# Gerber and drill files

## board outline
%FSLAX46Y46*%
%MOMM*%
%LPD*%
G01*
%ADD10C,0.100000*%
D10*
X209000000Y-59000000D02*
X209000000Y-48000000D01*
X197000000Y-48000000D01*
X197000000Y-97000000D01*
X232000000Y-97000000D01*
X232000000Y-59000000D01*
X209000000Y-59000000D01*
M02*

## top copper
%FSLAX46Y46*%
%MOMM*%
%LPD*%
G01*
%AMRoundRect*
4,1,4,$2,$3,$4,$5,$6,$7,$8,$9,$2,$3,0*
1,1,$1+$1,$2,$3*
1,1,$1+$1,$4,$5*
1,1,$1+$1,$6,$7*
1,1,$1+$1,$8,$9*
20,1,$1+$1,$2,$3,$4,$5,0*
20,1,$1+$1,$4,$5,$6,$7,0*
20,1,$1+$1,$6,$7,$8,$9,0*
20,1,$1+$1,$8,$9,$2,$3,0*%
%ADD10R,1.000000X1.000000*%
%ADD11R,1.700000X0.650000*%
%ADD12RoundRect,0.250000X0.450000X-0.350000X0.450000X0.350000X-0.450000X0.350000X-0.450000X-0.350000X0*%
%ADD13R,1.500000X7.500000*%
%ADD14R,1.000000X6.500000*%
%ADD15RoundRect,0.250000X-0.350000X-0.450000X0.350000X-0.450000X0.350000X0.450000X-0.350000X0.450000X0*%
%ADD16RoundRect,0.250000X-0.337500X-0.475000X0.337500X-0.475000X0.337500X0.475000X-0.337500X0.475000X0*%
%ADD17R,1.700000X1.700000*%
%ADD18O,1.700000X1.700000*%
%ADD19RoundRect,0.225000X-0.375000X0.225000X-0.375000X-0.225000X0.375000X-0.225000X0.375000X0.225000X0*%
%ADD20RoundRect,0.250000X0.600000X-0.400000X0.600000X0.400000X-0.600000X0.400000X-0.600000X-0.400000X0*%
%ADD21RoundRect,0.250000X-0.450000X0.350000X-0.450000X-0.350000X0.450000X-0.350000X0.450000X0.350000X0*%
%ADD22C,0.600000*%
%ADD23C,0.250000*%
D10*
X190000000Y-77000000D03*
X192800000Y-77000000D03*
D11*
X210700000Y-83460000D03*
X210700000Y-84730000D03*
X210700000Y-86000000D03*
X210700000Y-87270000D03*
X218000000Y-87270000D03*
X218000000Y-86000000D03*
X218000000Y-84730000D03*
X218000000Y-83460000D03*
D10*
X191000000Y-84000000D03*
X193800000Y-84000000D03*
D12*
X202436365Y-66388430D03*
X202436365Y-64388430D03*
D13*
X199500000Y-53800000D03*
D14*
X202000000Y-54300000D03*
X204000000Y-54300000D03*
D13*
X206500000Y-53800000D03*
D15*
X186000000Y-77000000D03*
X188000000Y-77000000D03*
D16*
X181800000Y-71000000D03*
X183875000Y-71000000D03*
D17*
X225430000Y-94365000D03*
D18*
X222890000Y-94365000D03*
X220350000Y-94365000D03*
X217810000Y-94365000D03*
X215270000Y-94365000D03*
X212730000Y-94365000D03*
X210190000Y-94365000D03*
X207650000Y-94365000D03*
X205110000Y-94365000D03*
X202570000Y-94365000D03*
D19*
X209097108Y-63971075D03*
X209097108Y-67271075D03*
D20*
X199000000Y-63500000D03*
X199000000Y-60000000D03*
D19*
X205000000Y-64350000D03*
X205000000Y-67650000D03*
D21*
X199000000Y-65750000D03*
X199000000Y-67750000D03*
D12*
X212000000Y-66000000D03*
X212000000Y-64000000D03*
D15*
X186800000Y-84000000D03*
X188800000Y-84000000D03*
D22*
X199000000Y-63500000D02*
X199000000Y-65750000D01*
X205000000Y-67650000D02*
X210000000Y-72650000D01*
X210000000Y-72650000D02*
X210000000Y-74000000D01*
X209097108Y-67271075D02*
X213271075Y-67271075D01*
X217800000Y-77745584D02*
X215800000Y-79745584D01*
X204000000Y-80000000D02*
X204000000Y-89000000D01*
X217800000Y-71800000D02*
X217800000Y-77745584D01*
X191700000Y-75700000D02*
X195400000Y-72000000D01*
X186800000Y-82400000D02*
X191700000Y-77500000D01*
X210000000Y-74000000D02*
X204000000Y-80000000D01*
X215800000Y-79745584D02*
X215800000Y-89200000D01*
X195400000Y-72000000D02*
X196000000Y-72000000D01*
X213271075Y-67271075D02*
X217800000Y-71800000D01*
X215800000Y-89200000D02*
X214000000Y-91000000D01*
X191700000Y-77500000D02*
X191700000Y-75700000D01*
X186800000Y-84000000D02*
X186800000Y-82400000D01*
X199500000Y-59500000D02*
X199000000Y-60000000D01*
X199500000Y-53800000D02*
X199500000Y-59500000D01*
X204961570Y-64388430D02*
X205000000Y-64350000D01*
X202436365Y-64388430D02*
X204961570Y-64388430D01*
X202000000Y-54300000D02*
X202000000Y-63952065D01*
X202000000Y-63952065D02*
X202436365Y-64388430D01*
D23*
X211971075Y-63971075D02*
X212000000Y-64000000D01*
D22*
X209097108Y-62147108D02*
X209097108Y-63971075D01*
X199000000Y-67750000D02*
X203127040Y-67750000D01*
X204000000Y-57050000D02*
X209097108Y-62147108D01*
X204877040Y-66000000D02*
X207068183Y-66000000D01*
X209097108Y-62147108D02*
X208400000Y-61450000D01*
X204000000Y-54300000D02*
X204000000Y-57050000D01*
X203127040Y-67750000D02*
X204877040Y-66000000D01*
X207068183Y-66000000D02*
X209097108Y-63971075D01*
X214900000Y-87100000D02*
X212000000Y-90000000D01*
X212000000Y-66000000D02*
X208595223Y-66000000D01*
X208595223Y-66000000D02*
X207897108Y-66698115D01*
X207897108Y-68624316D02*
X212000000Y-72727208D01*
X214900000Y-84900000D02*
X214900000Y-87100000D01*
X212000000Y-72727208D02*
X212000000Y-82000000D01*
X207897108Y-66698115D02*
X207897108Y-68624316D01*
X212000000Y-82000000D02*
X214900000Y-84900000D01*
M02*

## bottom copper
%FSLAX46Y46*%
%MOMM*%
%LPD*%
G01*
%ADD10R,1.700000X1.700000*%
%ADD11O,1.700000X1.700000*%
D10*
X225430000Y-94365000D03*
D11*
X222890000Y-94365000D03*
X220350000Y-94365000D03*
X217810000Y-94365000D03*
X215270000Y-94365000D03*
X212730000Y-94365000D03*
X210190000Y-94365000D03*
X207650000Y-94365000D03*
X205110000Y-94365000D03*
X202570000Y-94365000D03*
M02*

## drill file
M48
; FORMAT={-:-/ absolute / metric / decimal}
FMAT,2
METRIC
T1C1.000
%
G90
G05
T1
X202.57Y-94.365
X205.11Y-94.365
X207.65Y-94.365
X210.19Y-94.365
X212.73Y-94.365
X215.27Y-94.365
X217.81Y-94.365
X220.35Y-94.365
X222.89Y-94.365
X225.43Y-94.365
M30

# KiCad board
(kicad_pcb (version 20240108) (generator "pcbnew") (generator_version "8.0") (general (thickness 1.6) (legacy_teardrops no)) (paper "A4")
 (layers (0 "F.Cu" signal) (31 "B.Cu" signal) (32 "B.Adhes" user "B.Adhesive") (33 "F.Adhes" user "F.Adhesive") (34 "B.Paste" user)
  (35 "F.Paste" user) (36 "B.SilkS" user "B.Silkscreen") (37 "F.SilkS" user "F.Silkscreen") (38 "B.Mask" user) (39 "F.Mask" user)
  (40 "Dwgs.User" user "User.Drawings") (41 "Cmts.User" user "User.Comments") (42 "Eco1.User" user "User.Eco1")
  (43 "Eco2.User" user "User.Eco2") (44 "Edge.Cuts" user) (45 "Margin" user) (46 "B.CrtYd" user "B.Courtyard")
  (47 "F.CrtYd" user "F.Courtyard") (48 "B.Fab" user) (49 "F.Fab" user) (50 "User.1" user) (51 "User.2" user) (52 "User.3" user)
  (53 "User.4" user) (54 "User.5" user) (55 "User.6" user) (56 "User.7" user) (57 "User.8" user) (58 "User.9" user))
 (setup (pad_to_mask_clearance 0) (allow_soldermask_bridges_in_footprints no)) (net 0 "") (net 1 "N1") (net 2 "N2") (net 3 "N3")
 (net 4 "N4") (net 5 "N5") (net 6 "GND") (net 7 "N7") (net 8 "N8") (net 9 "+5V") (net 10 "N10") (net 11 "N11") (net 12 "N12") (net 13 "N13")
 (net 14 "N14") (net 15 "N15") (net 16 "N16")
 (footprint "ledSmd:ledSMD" (layer "F.Cu") (at 191.8 77)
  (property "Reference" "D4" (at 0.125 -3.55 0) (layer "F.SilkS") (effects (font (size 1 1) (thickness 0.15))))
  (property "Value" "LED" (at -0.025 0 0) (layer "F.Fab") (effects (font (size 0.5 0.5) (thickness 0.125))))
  (pad "1" smd rect (at -1.8 0) (size 1 1) (layers "F.Cu" "F.Paste" "F.Mask") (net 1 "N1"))
  (pad "2" smd rect (at 1 0) (size 1 1) (layers "F.Cu" "F.Paste" "F.Mask") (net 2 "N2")))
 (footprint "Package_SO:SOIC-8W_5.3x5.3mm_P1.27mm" (layer "F.Cu") (at 214.35 85.365)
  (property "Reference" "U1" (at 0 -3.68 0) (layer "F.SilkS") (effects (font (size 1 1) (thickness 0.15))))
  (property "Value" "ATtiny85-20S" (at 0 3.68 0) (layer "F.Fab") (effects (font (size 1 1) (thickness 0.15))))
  (pad "1" smd rect (at -3.65 -1.905) (size 1.7 0.65) (layers "F.Cu" "F.Paste" "F.Mask") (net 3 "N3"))
  (pad "2" smd rect (at -3.65 -0.635) (size 1.7 0.65) (layers "F.Cu" "F.Paste" "F.Mask") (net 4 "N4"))
  (pad "3" smd rect (at -3.65 0.635) (size 1.7 0.65) (layers "F.Cu" "F.Paste" "F.Mask") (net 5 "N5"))
  (pad "4" smd rect (at -3.65 1.905) (size 1.7 0.65) (layers "F.Cu" "F.Paste" "F.Mask") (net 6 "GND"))
  (pad "5" smd rect (at 3.65 1.905) (size 1.7 0.65) (layers "F.Cu" "F.Paste" "F.Mask") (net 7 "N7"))
  (pad "6" smd rect (at 3.65 0.635) (size 1.7 0.65) (layers "F.Cu" "F.Paste" "F.Mask") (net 2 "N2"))
  (pad "7" smd rect (at 3.65 -0.635) (size 1.7 0.65) (layers "F.Cu" "F.Paste" "F.Mask") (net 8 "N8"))
  (pad "8" smd rect (at 3.65 -1.905) (size 1.7 0.65) (layers "F.Cu" "F.Paste" "F.Mask") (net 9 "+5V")))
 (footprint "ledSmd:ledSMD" (layer "F.Cu") (at 192.8 84)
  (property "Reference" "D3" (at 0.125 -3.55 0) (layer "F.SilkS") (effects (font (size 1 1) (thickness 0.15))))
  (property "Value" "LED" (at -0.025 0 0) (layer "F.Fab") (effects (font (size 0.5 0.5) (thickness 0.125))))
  (pad "1" smd rect (at -1.8 0) (size 1 1) (layers "F.Cu" "F.Paste" "F.Mask") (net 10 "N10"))
  (pad "2" smd rect (at 1 0) (size 1 1) (layers "F.Cu" "F.Paste" "F.Mask") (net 9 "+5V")))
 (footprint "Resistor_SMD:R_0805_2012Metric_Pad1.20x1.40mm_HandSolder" (layer "F.Cu") (at 202.436365 65.38843 90)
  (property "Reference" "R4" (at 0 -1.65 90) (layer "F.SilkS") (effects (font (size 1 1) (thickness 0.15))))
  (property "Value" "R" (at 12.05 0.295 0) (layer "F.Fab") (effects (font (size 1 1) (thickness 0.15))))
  (pad "1" smd roundrect (at -1 0 90) (size 1.2 1.4) (layers "F.Cu" "F.Paste" "F.Mask") (roundrect_rratio 0.208333) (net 4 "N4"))
  (pad "2" smd roundrect (at 1 0 90) (size 1.2 1.4) (layers "F.Cu" "F.Paste" "F.Mask") (roundrect_rratio 0.208333) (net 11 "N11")))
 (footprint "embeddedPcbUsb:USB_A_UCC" (layer "F.Cu") (at 203 54 -90)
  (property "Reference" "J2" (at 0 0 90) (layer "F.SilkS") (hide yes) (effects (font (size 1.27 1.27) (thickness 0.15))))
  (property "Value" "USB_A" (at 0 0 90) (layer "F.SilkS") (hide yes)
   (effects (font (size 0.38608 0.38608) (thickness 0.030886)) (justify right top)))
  (pad "1" smd rect (at -0.2 3.5 270) (size 7.5 1.5) (layers "F.Cu" "F.Paste" "F.Mask") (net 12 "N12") (solder_mask_margin 0.1016))
  (pad "2" smd rect (at 0.3 1 270) (size 6.5 1) (layers "F.Cu" "F.Paste" "F.Mask") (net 11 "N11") (solder_mask_margin 0.1016))
  (pad "3" smd rect (at 0.3 -1 270) (size 6.5 1) (layers "F.Cu" "F.Paste" "F.Mask") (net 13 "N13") (solder_mask_margin 0.1016))
  (pad "4" smd rect (at -0.2 -3.5 270) (size 7.5 1.5) (layers "F.Cu" "F.Paste" "F.Mask") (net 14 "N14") (solder_mask_margin 0.1016)))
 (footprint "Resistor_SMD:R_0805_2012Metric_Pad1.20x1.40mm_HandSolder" (layer "F.Cu") (at 187 77)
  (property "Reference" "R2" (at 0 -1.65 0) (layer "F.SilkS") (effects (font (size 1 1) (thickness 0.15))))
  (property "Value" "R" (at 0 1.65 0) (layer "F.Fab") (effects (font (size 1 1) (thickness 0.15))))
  (pad "1" smd roundrect (at -1 0) (size 1.2 1.4) (layers "F.Cu" "F.Paste" "F.Mask") (roundrect_rratio 0.208333) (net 6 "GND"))
  (pad "2" smd roundrect (at 1 0) (size 1.2 1.4) (layers "F.Cu" "F.Paste" "F.Mask") (roundrect_rratio 0.208333) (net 1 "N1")))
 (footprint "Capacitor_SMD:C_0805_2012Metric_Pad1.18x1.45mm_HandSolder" (layer "F.Cu") (at 182.8375 71)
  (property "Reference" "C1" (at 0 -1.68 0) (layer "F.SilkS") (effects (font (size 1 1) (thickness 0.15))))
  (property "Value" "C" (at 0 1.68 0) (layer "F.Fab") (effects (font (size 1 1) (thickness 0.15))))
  (pad "1" smd roundrect (at -1.0375 0) (size 1.175 1.45) (layers "F.Cu" "F.Paste" "F.Mask") (roundrect_rratio 0.212766) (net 9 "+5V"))
  (pad "2" smd roundrect (at 1.0375 0) (size 1.175 1.45) (layers "F.Cu" "F.Paste" "F.Mask") (roundrect_rratio 0.212766) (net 6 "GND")))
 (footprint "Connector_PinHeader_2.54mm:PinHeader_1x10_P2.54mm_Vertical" (layer "F.Cu") (at 225.43 94.365 -90)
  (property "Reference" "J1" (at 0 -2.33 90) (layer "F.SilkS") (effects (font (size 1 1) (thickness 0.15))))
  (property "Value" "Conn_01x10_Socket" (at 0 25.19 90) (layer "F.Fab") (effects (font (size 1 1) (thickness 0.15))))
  (pad "1" thru_hole rect (at 0 0 270) (size 1.7 1.7) (drill 1) (layers "*.Cu" "*.Mask") (remove_unused_layers no) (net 9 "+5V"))
  (pad "2" thru_hole oval (at 0 2.54 270) (size 1.7 1.7) (drill 1) (layers "*.Cu" "*.Mask") (remove_unused_layers no) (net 6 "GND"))
  (pad "3" thru_hole oval (at 0 5.08 270) (size 1.7 1.7) (drill 1) (layers "*.Cu" "*.Mask") (remove_unused_layers no) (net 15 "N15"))
  (pad "4" thru_hole oval (at 0 7.62 270) (size 1.7 1.7) (drill 1) (layers "*.Cu" "*.Mask") (remove_unused_layers no) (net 7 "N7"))
  (pad "5" thru_hole oval (at 0 10.16 270) (size 1.7 1.7) (drill 1) (layers "*.Cu" "*.Mask") (remove_unused_layers no) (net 2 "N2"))
  (pad "6" thru_hole oval (at 0 12.7 270) (size 1.7 1.7) (drill 1) (layers "*.Cu" "*.Mask") (remove_unused_layers no) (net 8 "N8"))
  (pad "7" thru_hole oval (at 0 15.24 270) (size 1.7 1.7) (drill 1) (layers "*.Cu" "*.Mask") (remove_unused_layers no) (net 4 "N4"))
  (pad "8" thru_hole oval (at 0 17.78 270) (size 1.7 1.7) (drill 1) (layers "*.Cu" "*.Mask") (remove_unused_layers no) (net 5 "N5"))
  (pad "9" thru_hole oval (at 0 20.32 270) (size 1.7 1.7) (drill 1) (layers "*.Cu" "*.Mask") (remove_unused_layers no) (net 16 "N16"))
  (pad "10" thru_hole oval (at 0 22.86 270) (size 1.7 1.7) (drill 1) (layers "*.Cu" "*.Mask") (remove_unused_layers no) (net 3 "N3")))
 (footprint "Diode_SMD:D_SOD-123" (layer "F.Cu") (at 209.097108 65.621075 -90)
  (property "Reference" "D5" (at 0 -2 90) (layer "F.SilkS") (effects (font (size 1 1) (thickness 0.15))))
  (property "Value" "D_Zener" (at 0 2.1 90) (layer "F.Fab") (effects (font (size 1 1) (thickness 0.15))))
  (pad "1" smd roundrect (at -1.65 0 270) (size 0.9 1.2) (layers "F.Cu" "F.Paste" "F.Mask") (roundrect_rratio 0.25) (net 13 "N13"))
  (pad "2" smd roundrect (at 1.65 0 270) (size 0.9 1.2) (layers "F.Cu" "F.Paste" "F.Mask") (roundrect_rratio 0.25) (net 6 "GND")))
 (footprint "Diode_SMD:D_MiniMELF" (layer "F.Cu") (at 199 61.75 90)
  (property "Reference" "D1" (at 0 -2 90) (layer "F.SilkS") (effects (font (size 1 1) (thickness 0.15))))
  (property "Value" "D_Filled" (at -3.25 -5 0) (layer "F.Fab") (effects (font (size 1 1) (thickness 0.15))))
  (pad "1" smd roundrect (at -1.75 0 90) (size 1.3 1.7) (layers "F.Cu" "F.Paste" "F.Mask") (roundrect_rratio 0.1923076923) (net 9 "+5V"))
  (pad "2" smd roundrect (at 1.75 0 90) (size 1.3 1.7) (layers "F.Cu" "F.Paste" "F.Mask") (roundrect_rratio 0.1923076923) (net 12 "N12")))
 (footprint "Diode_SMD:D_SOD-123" (layer "F.Cu") (at 205 66 -90)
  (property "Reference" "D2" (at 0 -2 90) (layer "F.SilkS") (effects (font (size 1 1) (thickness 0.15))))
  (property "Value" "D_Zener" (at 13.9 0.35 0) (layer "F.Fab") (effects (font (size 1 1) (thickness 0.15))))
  (pad "1" smd roundrect (at -1.65 0 270) (size 0.9 1.2) (layers "F.Cu" "F.Paste" "F.Mask") (roundrect_rratio 0.25) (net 11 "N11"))
  (pad "2" smd roundrect (at 1.65 0 270) (size 0.9 1.2) (layers "F.Cu" "F.Paste" "F.Mask") (roundrect_rratio 0.25) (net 6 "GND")))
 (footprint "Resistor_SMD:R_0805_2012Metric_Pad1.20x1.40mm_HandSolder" (layer "F.Cu") (at 199 66.75 -90)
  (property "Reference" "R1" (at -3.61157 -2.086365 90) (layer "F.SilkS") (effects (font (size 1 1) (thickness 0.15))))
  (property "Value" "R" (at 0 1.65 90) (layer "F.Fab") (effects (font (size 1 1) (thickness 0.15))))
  (pad "1" smd roundrect (at -1 0 270) (size 1.2 1.4) (layers "F.Cu" "F.Paste" "F.Mask") (roundrect_rratio 0.208333) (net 9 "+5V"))
  (pad "2" smd roundrect (at 1 0 270) (size 1.2 1.4) (layers "F.Cu" "F.Paste" "F.Mask") (roundrect_rratio 0.208333) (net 13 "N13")))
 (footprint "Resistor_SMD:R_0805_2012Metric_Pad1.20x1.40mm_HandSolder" (layer "F.Cu") (at 212 65 90)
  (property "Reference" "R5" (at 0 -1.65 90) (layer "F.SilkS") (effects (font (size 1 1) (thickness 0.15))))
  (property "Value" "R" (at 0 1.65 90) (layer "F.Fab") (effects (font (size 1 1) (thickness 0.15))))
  (pad "1" smd roundrect (at -1 0 90) (size 1.2 1.4) (layers "F.Cu" "F.Paste" "F.Mask") (roundrect_rratio 0.208333) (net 8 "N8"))
  (pad "2" smd roundrect (at 1 0 90) (size 1.2 1.4) (layers "F.Cu" "F.Paste" "F.Mask") (roundrect_rratio 0.208333) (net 13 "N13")))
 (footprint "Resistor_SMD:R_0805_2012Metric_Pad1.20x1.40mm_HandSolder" (layer "F.Cu") (at 187.8 84)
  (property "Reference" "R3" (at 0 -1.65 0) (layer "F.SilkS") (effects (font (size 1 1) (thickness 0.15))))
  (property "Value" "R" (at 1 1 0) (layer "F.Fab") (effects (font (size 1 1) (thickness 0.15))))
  (pad "1" smd roundrect (at -1 0) (size 1.2 1.4) (layers "F.Cu" "F.Paste" "F.Mask") (roundrect_rratio 0.208333) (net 6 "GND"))
  (pad "2" smd roundrect (at 1 0) (size 1.2 1.4) (layers "F.Cu" "F.Paste" "F.Mask") (roundrect_rratio 0.208333) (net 10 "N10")))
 (gr_poly
  (pts (xy 209 59) (xy 209 48) (xy 197 48) (xy 197 97) (xy 232 97) (xy 232 59)) (stroke (width 0.1) (type solid)) (fill none)
  (layer "Edge.Cuts"))
 (segment (start 199 63.5) (end 199 65.75) (width 0.6) (layer "F.Cu") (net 9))
 (segment (start 205 67.65) (end 210 72.65) (width 0.6) (layer "F.Cu") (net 6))
 (segment (start 210 72.65) (end 210 74) (width 0.6) (layer "F.Cu") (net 6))
 (segment (start 209.097108 67.271075) (end 213.271075 67.271075) (width 0.6) (layer "F.Cu") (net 6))
 (segment (start 217.8 77.745584) (end 215.8 79.745584) (width 0.6) (layer "F.Cu") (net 6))
 (segment (start 204 80) (end 204 89) (width 0.6) (layer "F.Cu") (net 6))
 (segment (start 217.8 71.8) (end 217.8 77.745584) (width 0.6) (layer "F.Cu") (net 6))
 (segment (start 191.7 75.7) (end 195.4 72) (width 0.6) (layer "F.Cu") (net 6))
 (segment (start 186.8 82.4) (end 191.7 77.5) (width 0.6) (layer "F.Cu") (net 6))
 (segment (start 210 74) (end 204 80) (width 0.6) (layer "F.Cu") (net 6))
 (segment (start 215.8 79.745584) (end 215.8 89.2) (width 0.6) (layer "F.Cu") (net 6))
 (segment (start 195.4 72) (end 196 72) (width 0.6) (layer "F.Cu") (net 6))
 (segment (start 213.271075 67.271075) (end 217.8 71.8) (width 0.6) (layer "F.Cu") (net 6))
 (segment (start 215.8 89.2) (end 214 91) (width 0.6) (layer "F.Cu") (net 6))
 (segment (start 191.7 77.5) (end 191.7 75.7) (width 0.6) (layer "F.Cu") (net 6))
 (segment (start 186.8 84) (end 186.8 82.4) (width 0.6) (layer "F.Cu") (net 6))
 (segment (start 199.5 59.5) (end 199 60) (width 0.6) (layer "F.Cu") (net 12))
 (segment (start 199.5 53.8) (end 199.5 59.5) (width 0.6) (layer "F.Cu") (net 12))
 (segment (start 204.96157 64.38843) (end 205 64.35) (width 0.6) (layer "F.Cu") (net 11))
 (segment (start 202.436365 64.38843) (end 204.96157 64.38843) (width 0.6) (layer "F.Cu") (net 11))
 (segment (start 202 54.3) (end 202 63.952065) (width 0.6) (layer "F.Cu") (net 11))
 (segment (start 202 63.952065) (end 202.436365 64.38843) (width 0.6) (layer "F.Cu") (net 11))
 (segment (start 211.971075 63.971075) (end 212 64) (width 0.25) (layer "F.Cu") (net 13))
 (segment (start 209.097108 62.147108) (end 209.097108 63.971075) (width 0.6) (layer "F.Cu") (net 13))
 (segment (start 199 67.75) (end 203.12704 67.75) (width 0.6) (layer "F.Cu") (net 13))
 (segment (start 204 57.05) (end 209.097108 62.147108) (width 0.6) (layer "F.Cu") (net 13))
 (segment (start 204.87704 66) (end 207.068183 66) (width 0.6) (layer "F.Cu") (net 13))
 (segment (start 209.097108 62.147108) (end 208.4 61.45) (width 0.6) (layer "F.Cu") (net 13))
 (segment (start 204 54.3) (end 204 57.05) (width 0.6) (layer "F.Cu") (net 13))
 (segment (start 203.12704 67.75) (end 204.87704 66) (width 0.6) (layer "F.Cu") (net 13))
 (segment (start 207.068183 66) (end 209.097108 63.971075) (width 0.6) (layer "F.Cu") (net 13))
 (segment (start 214.9 87.1) (end 212 90) (width 0.6) (layer "F.Cu") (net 8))
 (segment (start 212 66) (end 208.595223 66) (width 0.6) (layer "F.Cu") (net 8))
 (segment (start 208.595223 66) (end 207.897108 66.698115) (width 0.6) (layer "F.Cu") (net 8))
 (segment (start 207.897108 68.624316) (end 212 72.727208) (width 0.6) (layer "F.Cu") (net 8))
 (segment (start 214.9 84.9) (end 214.9 87.1) (width 0.6) (layer "F.Cu") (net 8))
 (segment (start 212 72.727208) (end 212 82) (width 0.6) (layer "F.Cu") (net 8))
 (segment (start 207.897108 66.698115) (end 207.897108 68.624316) (width 0.6) (layer "F.Cu") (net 8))
 (segment (start 212 82) (end 214.9 84.9) (width 0.6) (layer "F.Cu") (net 8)))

